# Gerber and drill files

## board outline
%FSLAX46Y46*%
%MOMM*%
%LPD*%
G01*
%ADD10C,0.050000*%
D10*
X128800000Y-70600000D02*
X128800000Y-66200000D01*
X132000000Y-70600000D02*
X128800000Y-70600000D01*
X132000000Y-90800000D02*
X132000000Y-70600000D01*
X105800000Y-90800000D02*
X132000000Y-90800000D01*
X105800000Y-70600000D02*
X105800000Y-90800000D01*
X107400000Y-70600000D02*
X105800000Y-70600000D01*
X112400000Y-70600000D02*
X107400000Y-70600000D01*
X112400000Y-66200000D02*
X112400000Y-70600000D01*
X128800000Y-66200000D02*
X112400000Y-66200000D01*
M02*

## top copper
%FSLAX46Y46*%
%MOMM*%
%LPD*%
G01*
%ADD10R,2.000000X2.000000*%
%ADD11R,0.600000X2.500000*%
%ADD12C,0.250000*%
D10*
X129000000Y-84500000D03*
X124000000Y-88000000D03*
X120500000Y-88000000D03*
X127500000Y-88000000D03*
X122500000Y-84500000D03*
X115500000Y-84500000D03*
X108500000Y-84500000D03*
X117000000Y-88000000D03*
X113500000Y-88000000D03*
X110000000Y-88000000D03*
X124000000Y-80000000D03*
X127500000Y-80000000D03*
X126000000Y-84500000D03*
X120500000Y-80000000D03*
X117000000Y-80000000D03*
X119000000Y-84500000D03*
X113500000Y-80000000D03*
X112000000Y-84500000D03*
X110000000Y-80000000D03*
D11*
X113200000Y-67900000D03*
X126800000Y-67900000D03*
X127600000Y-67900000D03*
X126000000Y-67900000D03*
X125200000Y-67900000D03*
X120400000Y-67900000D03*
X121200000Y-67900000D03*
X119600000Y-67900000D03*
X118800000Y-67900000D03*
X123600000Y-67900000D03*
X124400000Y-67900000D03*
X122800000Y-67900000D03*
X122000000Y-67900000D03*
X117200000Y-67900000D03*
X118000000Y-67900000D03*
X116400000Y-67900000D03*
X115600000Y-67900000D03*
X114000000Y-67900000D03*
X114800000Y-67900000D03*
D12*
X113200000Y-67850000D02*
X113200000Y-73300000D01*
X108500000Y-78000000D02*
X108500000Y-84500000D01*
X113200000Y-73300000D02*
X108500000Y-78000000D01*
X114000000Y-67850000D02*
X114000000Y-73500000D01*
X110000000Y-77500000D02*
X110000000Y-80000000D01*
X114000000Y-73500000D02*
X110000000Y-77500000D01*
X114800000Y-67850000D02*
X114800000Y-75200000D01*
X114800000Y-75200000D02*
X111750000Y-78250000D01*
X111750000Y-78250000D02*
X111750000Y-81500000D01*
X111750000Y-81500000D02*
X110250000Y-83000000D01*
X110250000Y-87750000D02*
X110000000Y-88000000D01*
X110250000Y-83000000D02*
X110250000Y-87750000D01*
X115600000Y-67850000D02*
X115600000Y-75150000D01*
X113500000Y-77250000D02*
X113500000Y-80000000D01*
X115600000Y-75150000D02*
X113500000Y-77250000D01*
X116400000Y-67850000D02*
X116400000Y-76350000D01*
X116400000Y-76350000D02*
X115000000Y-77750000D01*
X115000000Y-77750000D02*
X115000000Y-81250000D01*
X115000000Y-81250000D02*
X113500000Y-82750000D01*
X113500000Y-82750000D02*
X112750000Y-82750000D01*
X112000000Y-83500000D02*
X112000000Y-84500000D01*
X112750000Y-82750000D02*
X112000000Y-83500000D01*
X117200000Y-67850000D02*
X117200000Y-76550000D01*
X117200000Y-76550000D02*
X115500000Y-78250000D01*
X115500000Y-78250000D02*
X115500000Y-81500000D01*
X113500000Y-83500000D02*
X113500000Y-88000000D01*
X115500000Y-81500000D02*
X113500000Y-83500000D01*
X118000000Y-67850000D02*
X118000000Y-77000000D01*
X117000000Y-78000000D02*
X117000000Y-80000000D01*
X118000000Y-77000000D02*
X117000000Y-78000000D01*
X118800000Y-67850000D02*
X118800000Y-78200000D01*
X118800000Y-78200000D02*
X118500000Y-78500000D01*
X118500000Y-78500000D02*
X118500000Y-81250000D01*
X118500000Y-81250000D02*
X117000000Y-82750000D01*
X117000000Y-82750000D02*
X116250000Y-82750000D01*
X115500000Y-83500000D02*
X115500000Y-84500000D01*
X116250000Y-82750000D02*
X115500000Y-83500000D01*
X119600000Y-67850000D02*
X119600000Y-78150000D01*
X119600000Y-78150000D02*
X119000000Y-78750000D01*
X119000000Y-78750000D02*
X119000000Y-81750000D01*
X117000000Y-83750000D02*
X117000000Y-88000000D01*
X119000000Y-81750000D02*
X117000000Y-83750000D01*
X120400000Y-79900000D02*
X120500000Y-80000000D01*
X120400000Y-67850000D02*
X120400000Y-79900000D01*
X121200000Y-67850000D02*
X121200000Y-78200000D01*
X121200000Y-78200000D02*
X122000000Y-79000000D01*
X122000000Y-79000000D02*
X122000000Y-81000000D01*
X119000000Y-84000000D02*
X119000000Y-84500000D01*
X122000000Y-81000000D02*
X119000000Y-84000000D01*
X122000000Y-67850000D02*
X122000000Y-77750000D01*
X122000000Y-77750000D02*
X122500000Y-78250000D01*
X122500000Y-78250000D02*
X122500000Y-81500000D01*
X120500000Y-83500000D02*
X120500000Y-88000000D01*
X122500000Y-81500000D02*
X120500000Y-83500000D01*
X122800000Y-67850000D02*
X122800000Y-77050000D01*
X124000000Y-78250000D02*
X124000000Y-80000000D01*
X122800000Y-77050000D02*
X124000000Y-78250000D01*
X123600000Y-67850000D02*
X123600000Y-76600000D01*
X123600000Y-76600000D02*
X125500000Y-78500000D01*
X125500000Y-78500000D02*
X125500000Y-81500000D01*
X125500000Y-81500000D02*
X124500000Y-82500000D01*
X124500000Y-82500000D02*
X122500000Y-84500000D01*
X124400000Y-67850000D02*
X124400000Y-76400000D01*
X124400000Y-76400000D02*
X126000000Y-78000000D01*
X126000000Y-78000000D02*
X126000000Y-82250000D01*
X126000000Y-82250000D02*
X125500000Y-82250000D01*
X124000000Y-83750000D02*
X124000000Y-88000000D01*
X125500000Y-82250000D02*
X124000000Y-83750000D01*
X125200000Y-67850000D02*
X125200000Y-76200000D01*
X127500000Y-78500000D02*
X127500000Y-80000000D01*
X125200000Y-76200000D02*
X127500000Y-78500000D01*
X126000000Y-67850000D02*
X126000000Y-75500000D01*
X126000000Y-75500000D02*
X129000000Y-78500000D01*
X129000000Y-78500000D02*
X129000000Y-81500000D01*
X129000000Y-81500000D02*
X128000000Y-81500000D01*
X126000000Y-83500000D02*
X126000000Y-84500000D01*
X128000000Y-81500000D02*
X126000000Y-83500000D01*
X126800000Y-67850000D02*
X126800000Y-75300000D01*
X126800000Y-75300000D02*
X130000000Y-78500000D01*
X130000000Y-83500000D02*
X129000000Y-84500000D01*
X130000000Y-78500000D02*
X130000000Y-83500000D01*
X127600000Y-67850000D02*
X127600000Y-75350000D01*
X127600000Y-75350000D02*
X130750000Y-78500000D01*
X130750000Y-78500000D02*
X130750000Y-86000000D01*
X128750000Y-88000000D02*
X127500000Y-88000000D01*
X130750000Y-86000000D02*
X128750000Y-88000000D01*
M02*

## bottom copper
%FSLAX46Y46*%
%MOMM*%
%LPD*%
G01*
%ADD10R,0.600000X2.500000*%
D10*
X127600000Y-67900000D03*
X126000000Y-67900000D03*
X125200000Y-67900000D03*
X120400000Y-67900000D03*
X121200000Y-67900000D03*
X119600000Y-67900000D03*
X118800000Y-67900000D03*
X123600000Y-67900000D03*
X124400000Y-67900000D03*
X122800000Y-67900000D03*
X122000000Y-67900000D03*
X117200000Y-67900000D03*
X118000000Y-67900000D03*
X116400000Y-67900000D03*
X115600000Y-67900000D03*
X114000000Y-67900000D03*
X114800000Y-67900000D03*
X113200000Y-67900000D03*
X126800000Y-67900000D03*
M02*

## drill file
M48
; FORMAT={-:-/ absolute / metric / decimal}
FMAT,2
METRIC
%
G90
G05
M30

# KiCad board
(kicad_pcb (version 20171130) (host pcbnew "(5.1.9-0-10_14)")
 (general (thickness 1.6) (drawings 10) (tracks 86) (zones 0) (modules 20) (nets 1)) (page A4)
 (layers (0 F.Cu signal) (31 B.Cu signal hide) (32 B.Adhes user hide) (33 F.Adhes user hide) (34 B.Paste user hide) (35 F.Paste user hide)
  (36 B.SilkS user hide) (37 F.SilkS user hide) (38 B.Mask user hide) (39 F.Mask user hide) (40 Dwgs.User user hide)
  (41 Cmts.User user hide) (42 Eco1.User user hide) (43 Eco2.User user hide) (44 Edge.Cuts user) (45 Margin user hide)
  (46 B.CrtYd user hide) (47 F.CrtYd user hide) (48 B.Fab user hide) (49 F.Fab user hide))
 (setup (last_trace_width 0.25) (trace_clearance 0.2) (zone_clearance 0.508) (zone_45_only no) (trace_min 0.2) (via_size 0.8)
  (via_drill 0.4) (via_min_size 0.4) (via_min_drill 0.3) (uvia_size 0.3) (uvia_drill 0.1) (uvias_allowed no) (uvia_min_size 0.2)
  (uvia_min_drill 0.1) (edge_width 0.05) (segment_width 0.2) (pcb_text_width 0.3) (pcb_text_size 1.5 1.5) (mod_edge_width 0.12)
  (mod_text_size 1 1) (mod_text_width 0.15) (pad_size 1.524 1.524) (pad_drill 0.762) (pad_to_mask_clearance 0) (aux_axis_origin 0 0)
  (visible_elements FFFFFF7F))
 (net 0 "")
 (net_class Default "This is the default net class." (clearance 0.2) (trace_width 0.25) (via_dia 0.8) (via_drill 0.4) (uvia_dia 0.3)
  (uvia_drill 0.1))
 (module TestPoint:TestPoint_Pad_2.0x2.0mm (layer F.Cu) (at 129 84.5)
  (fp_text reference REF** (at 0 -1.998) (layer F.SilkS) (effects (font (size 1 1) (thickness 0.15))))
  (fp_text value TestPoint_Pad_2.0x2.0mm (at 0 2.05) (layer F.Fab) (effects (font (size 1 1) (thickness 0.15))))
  (pad 1 smd rect (at 0 0) (size 2 2) (layers F.Cu F.Mask)))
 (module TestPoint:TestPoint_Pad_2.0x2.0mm (layer F.Cu) (at 124 88)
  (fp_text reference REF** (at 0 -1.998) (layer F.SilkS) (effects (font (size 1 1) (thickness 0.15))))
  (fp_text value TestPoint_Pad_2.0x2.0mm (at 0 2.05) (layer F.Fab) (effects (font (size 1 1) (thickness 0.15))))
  (pad 1 smd rect (at 0 0) (size 2 2) (layers F.Cu F.Mask)))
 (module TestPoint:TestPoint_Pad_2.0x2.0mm (layer F.Cu) (at 120.5 88)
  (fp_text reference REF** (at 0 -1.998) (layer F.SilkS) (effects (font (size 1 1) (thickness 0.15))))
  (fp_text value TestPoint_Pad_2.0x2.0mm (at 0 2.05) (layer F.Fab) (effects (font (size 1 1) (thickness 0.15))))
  (pad 1 smd rect (at 0 0) (size 2 2) (layers F.Cu F.Mask)))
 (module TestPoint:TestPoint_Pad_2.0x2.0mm (layer F.Cu) (at 127.5 88)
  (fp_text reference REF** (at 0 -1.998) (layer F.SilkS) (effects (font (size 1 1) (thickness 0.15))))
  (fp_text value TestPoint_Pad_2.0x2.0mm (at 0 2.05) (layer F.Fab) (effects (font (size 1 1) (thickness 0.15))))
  (pad 1 smd rect (at 0 0) (size 2 2) (layers F.Cu F.Mask)))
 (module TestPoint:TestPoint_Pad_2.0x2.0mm (layer F.Cu) (at 122.5 84.5)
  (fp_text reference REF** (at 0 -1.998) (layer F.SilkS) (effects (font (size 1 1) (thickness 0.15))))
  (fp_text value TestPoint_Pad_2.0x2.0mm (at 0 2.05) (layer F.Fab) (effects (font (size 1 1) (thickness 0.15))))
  (pad 1 smd rect (at 0 0) (size 2 2) (layers F.Cu F.Mask)))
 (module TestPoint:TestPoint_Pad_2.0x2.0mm (layer F.Cu) (at 115.5 84.5)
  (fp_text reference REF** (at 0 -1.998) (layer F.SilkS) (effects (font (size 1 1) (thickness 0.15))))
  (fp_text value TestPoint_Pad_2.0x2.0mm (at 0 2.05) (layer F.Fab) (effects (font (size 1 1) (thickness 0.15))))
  (pad 1 smd rect (at 0 0) (size 2 2) (layers F.Cu F.Mask)))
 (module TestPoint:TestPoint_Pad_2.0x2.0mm (layer F.Cu) (at 108.5 84.5)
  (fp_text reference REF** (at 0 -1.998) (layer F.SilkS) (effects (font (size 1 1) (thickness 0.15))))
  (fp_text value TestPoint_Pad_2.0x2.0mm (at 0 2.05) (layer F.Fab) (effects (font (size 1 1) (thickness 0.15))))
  (pad 1 smd rect (at 0 0) (size 2 2) (layers F.Cu F.Mask)))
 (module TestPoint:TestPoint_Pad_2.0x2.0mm (layer F.Cu) (at 117 88)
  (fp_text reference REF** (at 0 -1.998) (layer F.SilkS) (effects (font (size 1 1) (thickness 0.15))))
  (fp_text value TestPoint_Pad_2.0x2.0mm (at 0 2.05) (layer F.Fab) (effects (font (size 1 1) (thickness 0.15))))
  (pad 1 smd rect (at 0 0) (size 2 2) (layers F.Cu F.Mask)))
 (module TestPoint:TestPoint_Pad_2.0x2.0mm (layer F.Cu) (at 113.5 88)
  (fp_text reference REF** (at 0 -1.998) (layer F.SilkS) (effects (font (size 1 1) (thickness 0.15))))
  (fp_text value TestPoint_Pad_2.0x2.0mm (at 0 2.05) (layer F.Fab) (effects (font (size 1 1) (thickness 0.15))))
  (pad 1 smd rect (at 0 0) (size 2 2) (layers F.Cu F.Mask)))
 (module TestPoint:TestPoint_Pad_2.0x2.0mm (layer F.Cu) (at 110 88)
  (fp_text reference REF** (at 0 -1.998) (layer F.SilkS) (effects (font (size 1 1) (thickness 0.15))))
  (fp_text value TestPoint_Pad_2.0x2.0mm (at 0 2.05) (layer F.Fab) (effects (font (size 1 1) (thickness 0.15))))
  (pad 1 smd rect (at 0 0) (size 2 2) (layers F.Cu F.Mask)))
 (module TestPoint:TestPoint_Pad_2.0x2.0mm (layer F.Cu) (at 124 80)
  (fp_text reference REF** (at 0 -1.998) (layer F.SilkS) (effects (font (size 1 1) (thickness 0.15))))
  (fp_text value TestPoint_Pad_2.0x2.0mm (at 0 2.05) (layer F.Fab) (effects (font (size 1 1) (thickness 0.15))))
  (pad 1 smd rect (at 0 0) (size 2 2) (layers F.Cu F.Mask)))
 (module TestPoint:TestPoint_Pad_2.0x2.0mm (layer F.Cu) (at 127.5 80)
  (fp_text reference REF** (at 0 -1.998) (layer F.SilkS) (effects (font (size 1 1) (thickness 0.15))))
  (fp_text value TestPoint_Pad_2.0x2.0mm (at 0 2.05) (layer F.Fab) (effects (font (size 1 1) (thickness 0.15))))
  (pad 1 smd rect (at 0 0) (size 2 2) (layers F.Cu F.Mask)))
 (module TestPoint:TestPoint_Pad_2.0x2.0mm (layer F.Cu) (at 126 84.5)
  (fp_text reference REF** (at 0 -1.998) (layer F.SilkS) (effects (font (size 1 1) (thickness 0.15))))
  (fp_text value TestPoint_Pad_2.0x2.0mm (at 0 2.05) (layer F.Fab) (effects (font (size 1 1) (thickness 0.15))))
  (pad 1 smd rect (at 0 0) (size 2 2) (layers F.Cu F.Mask)))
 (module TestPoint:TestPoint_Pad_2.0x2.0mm (layer F.Cu) (at 120.5 80)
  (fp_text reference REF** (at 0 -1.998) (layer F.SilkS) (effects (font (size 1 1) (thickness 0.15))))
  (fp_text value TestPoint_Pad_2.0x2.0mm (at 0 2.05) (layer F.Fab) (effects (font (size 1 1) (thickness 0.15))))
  (pad 1 smd rect (at 0 0) (size 2 2) (layers F.Cu F.Mask)))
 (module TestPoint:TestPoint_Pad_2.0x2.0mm (layer F.Cu) (at 117 80)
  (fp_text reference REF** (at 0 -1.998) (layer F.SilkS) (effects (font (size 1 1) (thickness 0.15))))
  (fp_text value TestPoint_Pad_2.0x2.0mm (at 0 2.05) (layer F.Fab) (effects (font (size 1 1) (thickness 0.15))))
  (pad 1 smd rect (at 0 0) (size 2 2) (layers F.Cu F.Mask)))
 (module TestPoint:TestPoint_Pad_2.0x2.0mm (layer F.Cu) (at 119 84.5)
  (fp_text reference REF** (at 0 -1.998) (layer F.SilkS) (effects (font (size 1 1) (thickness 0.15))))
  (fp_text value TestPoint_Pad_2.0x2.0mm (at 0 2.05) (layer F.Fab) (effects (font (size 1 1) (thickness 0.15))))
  (pad 1 smd rect (at 0 0) (size 2 2) (layers F.Cu F.Mask)))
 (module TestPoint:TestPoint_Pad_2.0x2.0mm (layer F.Cu) (at 113.5 80)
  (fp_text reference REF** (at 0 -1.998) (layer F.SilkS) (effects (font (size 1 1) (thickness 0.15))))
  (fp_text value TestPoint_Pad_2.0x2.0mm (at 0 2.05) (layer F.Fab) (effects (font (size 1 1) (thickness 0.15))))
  (pad 1 smd rect (at 0 0) (size 2 2) (layers F.Cu F.Mask)))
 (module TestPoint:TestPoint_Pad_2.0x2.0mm (layer F.Cu) (at 112 84.5)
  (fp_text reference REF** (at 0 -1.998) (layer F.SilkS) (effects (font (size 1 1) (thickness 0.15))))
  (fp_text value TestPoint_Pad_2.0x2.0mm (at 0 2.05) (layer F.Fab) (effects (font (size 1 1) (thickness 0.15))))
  (pad 1 smd rect (at 0 0) (size 2 2) (layers F.Cu F.Mask)))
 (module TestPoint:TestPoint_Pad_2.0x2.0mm (layer F.Cu) (at 110 80)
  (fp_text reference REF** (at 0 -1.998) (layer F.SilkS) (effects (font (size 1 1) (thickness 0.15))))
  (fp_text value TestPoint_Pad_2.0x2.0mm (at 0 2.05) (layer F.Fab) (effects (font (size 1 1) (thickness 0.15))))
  (pad 1 smd rect (at 0 0) (size 2 2) (layers F.Cu F.Mask)))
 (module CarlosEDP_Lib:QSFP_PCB (layer F.Cu) (at 112.8 69.45)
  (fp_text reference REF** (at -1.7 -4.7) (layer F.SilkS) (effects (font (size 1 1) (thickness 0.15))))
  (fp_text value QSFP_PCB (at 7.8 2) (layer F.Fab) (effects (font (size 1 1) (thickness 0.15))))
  (pad 1 smd rect (at 14.8 -1.5) (size 0.6 2.5) (drill (offset 0 -0.05)) (layers B.Cu B.Paste B.Mask))
  (pad 3 smd rect (at 13.2 -1.5) (size 0.6 2.5) (drill (offset 0 -0.05)) (layers B.Cu B.Paste B.Mask))
  (pad 4 smd rect (at 12.4 -1.5) (size 0.6 2.5) (drill (offset 0 -0.05)) (layers B.Cu B.Paste B.Mask))
  (pad 10 smd rect (at 7.6 -1.5) (size 0.6 2.5) (drill (offset 0 -0.05)) (layers B.Cu B.Paste B.Mask))
  (pad 9 smd rect (at 8.4 -1.5) (size 0.6 2.5) (drill (offset 0 -0.05)) (layers B.Cu B.Paste B.Mask))
  (pad 11 smd rect (at 6.8 -1.5) (size 0.6 2.5) (drill (offset 0 -0.05)) (layers B.Cu B.Paste B.Mask))
  (pad 12 smd rect (at 6 -1.5) (size 0.6 2.5) (drill (offset 0 -0.05)) (layers B.Cu B.Paste B.Mask))
  (pad 6 smd rect (at 10.8 -1.5) (size 0.6 2.5) (drill (offset 0 -0.05)) (layers B.Cu B.Paste B.Mask))
  (pad 5 smd rect (at 11.6 -1.5) (size 0.6 2.5) (drill (offset 0 -0.05)) (layers B.Cu B.Paste B.Mask))
  (pad 7 smd rect (at 10 -1.5) (size 0.6 2.5) (drill (offset 0 -0.05)) (layers B.Cu B.Paste B.Mask))
  (pad 8 smd rect (at 9.2 -1.5) (size 0.6 2.5) (drill (offset 0 -0.05)) (layers B.Cu B.Paste B.Mask))
  (pad 14 smd rect (at 4.4 -1.5) (size 0.6 2.5) (drill (offset 0 -0.05)) (layers B.Cu B.Paste B.Mask))
  (pad 13 smd rect (at 5.2 -1.5) (size 0.6 2.5) (drill (offset 0 -0.05)) (layers B.Cu B.Paste B.Mask))
  (pad 15 smd rect (at 3.6 -1.5) (size 0.6 2.5) (drill (offset 0 -0.05)) (layers B.Cu B.Paste B.Mask))
  (pad 16 smd rect (at 2.8 -1.5) (size 0.6 2.5) (drill (offset 0 -0.05)) (layers B.Cu B.Paste B.Mask))
  (pad 18 smd rect (at 1.2 -1.5) (size 0.6 2.5) (drill (offset 0 -0.05)) (layers B.Cu B.Paste B.Mask))
  (pad 17 smd rect (at 2 -1.5) (size 0.6 2.5) (drill (offset 0 -0.05)) (layers B.Cu B.Paste B.Mask))
  (pad 19 smd rect (at 0.4 -1.5) (size 0.6 2.5) (drill (offset 0 -0.05)) (layers B.Cu B.Paste B.Mask))
  (pad 2 smd rect (at 14 -1.5) (size 0.6 2.5) (drill (offset 0 -0.05)) (layers B.Cu B.Paste B.Mask))
  (pad 38 smd rect (at 0.4 -1.6) (size 0.6 2.5) (drill (offset 0 0.05)) (layers F.Cu F.Paste F.Mask))
  (pad 21 smd rect (at 14 -1.6) (size 0.6 2.5) (drill (offset 0 0.05)) (layers F.Cu F.Paste F.Mask))
  (pad 20 smd rect (at 14.8 -1.6) (size 0.6 2.5) (drill (offset 0 0.05)) (layers F.Cu F.Paste F.Mask))
  (pad 22 smd rect (at 13.2 -1.6) (size 0.6 2.5) (drill (offset 0 0.05)) (layers F.Cu F.Paste F.Mask))
  (pad 23 smd rect (at 12.4 -1.6) (size 0.6 2.5) (drill (offset 0 0.05)) (layers F.Cu F.Paste F.Mask))
  (pad 29 smd rect (at 7.6 -1.6) (size 0.6 2.5) (drill (offset 0 0.05)) (layers F.Cu F.Paste F.Mask))
  (pad 28 smd rect (at 8.4 -1.6) (size 0.6 2.5) (drill (offset 0 0.05)) (layers F.Cu F.Paste F.Mask))
  (pad 30 smd rect (at 6.8 -1.6) (size 0.6 2.5) (drill (offset 0 0.05)) (layers F.Cu F.Paste F.Mask))
  (pad 31 smd rect (at 6 -1.6) (size 0.6 2.5) (drill (offset 0 0.05)) (layers F.Cu F.Paste F.Mask))
  (pad 25 smd rect (at 10.8 -1.6) (size 0.6 2.5) (drill (offset 0 0.05)) (layers F.Cu F.Paste F.Mask))
  (pad 24 smd rect (at 11.6 -1.6) (size 0.6 2.5) (drill (offset 0 0.05)) (layers F.Cu F.Paste F.Mask))
  (pad 26 smd rect (at 10 -1.6) (size 0.6 2.5) (drill (offset 0 0.05)) (layers F.Cu F.Paste F.Mask))
  (pad 27 smd rect (at 9.2 -1.6) (size 0.6 2.5) (drill (offset 0 0.05)) (layers F.Cu F.Paste F.Mask))
  (pad 33 smd rect (at 4.4 -1.6) (size 0.6 2.5) (drill (offset 0 0.05)) (layers F.Cu F.Paste F.Mask))
  (pad 32 smd rect (at 5.2 -1.6) (size 0.6 2.5) (drill (offset 0 0.05)) (layers F.Cu F.Paste F.Mask))
  (pad 34 smd rect (at 3.6 -1.6) (size 0.6 2.5) (drill (offset 0 0.05)) (layers F.Cu F.Paste F.Mask))
  (pad 35 smd rect (at 2.8 -1.6) (size 0.6 2.5) (drill (offset 0 0.05)) (layers F.Cu F.Paste F.Mask))
  (pad 37 smd rect (at 1.2 -1.6) (size 0.6 2.5) (drill (offset 0 0.05)) (layers F.Cu F.Paste F.Mask))
  (pad 36 smd rect (at 2 -1.6) (size 0.6 2.5) (drill (offset 0 0.05)) (layers F.Cu F.Paste F.Mask)))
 (gr_line (start 128.8 70.6) (end 128.8 66.2) (layer Edge.Cuts) (width 0.05))
 (gr_line (start 132 70.6) (end 128.8 70.6) (layer Edge.Cuts) (width 0.05))
 (gr_line (start 132 90.8) (end 132 70.6) (layer Edge.Cuts) (width 0.05))
 (gr_line (start 105.8 90.8) (end 132 90.8) (layer Edge.Cuts) (width 0.05))
 (gr_line (start 105.8 70.6) (end 105.8 90.8) (layer Edge.Cuts) (width 0.05))
 (gr_line (start 107.4 70.6) (end 105.8 70.6) (layer Edge.Cuts) (width 0.05))
 (gr_line (start 112.4 70.6) (end 107.4 70.6) (layer Edge.Cuts) (width 0.05))
 (gr_line (start 112.4 66.2) (end 112.4 70.6) (layer Edge.Cuts) (width 0.05))
 (gr_line (start 128.8 66.2) (end 112.4 66.2) (layer Edge.Cuts) (width 0.05))
 (segment (start 113.2 67.85) (end 113.2 73.3) (width 0.25) (layer F.Cu) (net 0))
 (segment (start 108.5 78) (end 108.5 84.5) (width 0.25) (layer F.Cu) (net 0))
 (segment (start 113.2 73.3) (end 108.5 78) (width 0.25) (layer F.Cu) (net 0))
 (segment (start 114 67.85) (end 114 73.5) (width 0.25) (layer F.Cu) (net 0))
 (segment (start 110 77.5) (end 110 80) (width 0.25) (layer F.Cu) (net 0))
 (segment (start 114 73.5) (end 110 77.5) (width 0.25) (layer F.Cu) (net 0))
 (segment (start 114.8 67.85) (end 114.8 75.2) (width 0.25) (layer F.Cu) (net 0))
 (segment (start 114.8 75.2) (end 111.75 78.25) (width 0.25) (layer F.Cu) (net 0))
 (segment (start 111.75 78.25) (end 111.75 81.5) (width 0.25) (layer F.Cu) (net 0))
 (segment (start 111.75 81.5) (end 110.25 83) (width 0.25) (layer F.Cu) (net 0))
 (segment (start 110.25 87.75) (end 110 88) (width 0.25) (layer F.Cu) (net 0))
 (segment (start 110.25 83) (end 110.25 87.75) (width 0.25) (layer F.Cu) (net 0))
 (segment (start 115.6 67.85) (end 115.6 75.15) (width 0.25) (layer F.Cu) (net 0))
 (segment (start 113.5 77.25) (end 113.5 80) (width 0.25) (layer F.Cu) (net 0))
 (segment (start 115.6 75.15) (end 113.5 77.25) (width 0.25) (layer F.Cu) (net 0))
 (segment (start 116.4 67.85) (end 116.4 76.35) (width 0.25) (layer F.Cu) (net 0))
 (segment (start 116.4 76.35) (end 115 77.75) (width 0.25) (layer F.Cu) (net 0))
 (segment (start 115 77.75) (end 115 81.25) (width 0.25) (layer F.Cu) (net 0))
 (segment (start 115 81.25) (end 113.5 82.75) (width 0.25) (layer F.Cu) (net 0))
 (segment (start 113.5 82.75) (end 112.75 82.75) (width 0.25) (layer F.Cu) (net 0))
 (segment (start 112 83.5) (end 112 84.5) (width 0.25) (layer F.Cu) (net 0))
 (segment (start 112.75 82.75) (end 112 83.5) (width 0.25) (layer F.Cu) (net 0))
 (segment (start 117.2 67.85) (end 117.2 76.55) (width 0.25) (layer F.Cu) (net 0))
 (segment (start 117.2 76.55) (end 115.5 78.25) (width 0.25) (layer F.Cu) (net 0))
 (segment (start 115.5 78.25) (end 115.5 81.5) (width 0.25) (layer F.Cu) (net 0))
 (segment (start 113.5 83.5) (end 113.5 88) (width 0.25) (layer F.Cu) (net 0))
 (segment (start 115.5 81.5) (end 113.5 83.5) (width 0.25) (layer F.Cu) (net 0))
 (segment (start 118 67.85) (end 118 77) (width 0.25) (layer F.Cu) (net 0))
 (segment (start 117 78) (end 117 80) (width 0.25) (layer F.Cu) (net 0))
 (segment (start 118 77) (end 117 78) (width 0.25) (layer F.Cu) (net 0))
 (segment (start 118.8 67.85) (end 118.8 78.2) (width 0.25) (layer F.Cu) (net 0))
 (segment (start 118.8 78.2) (end 118.5 78.5) (width 0.25) (layer F.Cu) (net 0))
 (segment (start 118.5 78.5) (end 118.5 81.25) (width 0.25) (layer F.Cu) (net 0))
 (segment (start 118.5 81.25) (end 117 82.75) (width 0.25) (layer F.Cu) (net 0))
 (segment (start 117 82.75) (end 116.25 82.75) (width 0.25) (layer F.Cu) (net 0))
 (segment (start 115.5 83.5) (end 115.5 84.5) (width 0.25) (layer F.Cu) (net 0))
 (segment (start 116.25 82.75) (end 115.5 83.5) (width 0.25) (layer F.Cu) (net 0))
 (segment (start 119.6 67.85) (end 119.6 78.15) (width 0.25) (layer F.Cu) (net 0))
 (segment (start 119.6 78.15) (end 119 78.75) (width 0.25) (layer F.Cu) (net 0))
 (segment (start 119 78.75) (end 119 81.75) (width 0.25) (layer F.Cu) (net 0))
 (segment (start 117 83.75) (end 117 88) (width 0.25) (layer F.Cu) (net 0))
 (segment (start 119 81.75) (end 117 83.75) (width 0.25) (layer F.Cu) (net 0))
 (segment (start 120.4 79.9) (end 120.5 80) (width 0.25) (layer F.Cu) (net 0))
 (segment (start 120.4 67.85) (end 120.4 79.9) (width 0.25) (layer F.Cu) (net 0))
 (segment (start 121.2 67.85) (end 121.2 78.2) (width 0.25) (layer F.Cu) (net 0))
 (segment (start 121.2 78.2) (end 122 79) (width 0.25) (layer F.Cu) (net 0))
 (segment (start 122 79) (end 122 81) (width 0.25) (layer F.Cu) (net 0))
 (segment (start 119 84) (end 119 84.5) (width 0.25) (layer F.Cu) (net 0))
 (segment (start 122 81) (end 119 84) (width 0.25) (layer F.Cu) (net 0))
 (segment (start 122 67.85) (end 122 77.75) (width 0.25) (layer F.Cu) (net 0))
 (segment (start 122 77.75) (end 122.5 78.25) (width 0.25) (layer F.Cu) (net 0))
 (segment (start 122.5 78.25) (end 122.5 81.5) (width 0.25) (layer F.Cu) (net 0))
 (segment (start 120.5 83.5) (end 120.5 88) (width 0.25) (layer F.Cu) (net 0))
 (segment (start 122.5 81.5) (end 120.5 83.5) (width 0.25) (layer F.Cu) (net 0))
 (segment (start 122.8 67.85) (end 122.8 77.05) (width 0.25) (layer F.Cu) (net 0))
 (segment (start 124 78.25) (end 124 80) (width 0.25) (layer F.Cu) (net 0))
 (segment (start 122.8 77.05) (end 124 78.25) (width 0.25) (layer F.Cu) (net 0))
 (segment (start 123.6 67.85) (end 123.6 76.6) (width 0.25) (layer F.Cu) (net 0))
 (segment (start 123.6 76.6) (end 125.5 78.5) (width 0.25) (layer F.Cu) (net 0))
 (segment (start 125.5 78.5) (end 125.5 81.5) (width 0.25) (layer F.Cu) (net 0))
 (segment (start 125.5 81.5) (end 124.5 82.5) (width 0.25) (layer F.Cu) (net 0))
 (segment (start 124.5 82.5) (end 122.5 84.5) (width 0.25) (layer F.Cu) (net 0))
 (segment (start 124.4 67.85) (end 124.4 76.4) (width 0.25) (layer F.Cu) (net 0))
 (segment (start 124.4 76.4) (end 126 78) (width 0.25) (layer F.Cu) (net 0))
 (segment (start 126 78) (end 126 82.25) (width 0.25) (layer F.Cu) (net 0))
 (segment (start 126 82.25) (end 125.5 82.25) (width 0.25) (layer F.Cu) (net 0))
 (segment (start 124 83.75) (end 124 88) (width 0.25) (layer F.Cu) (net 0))
 (segment (start 125.5 82.25) (end 124 83.75) (width 0.25) (layer F.Cu) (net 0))
 (segment (start 125.2 67.85) (end 125.2 76.2) (width 0.25) (layer F.Cu) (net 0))
 (segment (start 127.5 78.5) (end 127.5 80) (width 0.25) (layer F.Cu) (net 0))
 (segment (start 125.2 76.2) (end 127.5 78.5) (width 0.25) (layer F.Cu) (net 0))
 (segment (start 126 67.85) (end 126 75.5) (width 0.25) (layer F.Cu) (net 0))
 (segment (start 126 75.5) (end 129 78.5) (width 0.25) (layer F.Cu) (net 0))
 (segment (start 129 78.5) (end 129 81.5) (width 0.25) (layer F.Cu) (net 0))
 (segment (start 129 81.5) (end 128 81.5) (width 0.25) (layer F.Cu) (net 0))
 (segment (start 126 83.5) (end 126 84.5) (width 0.25) (layer F.Cu) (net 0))
 (segment (start 128 81.5) (end 126 83.5) (width 0.25) (layer F.Cu) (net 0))
 (segment (start 126.8 67.85) (end 126.8 75.3) (width 0.25) (layer F.Cu) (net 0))
 (segment (start 126.8 75.3) (end 130 78.5) (width 0.25) (layer F.Cu) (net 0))
 (segment (start 130 83.5) (end 129 84.5) (width 0.25) (layer F.Cu) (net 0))
 (segment (start 130 78.5) (end 130 83.5) (width 0.25) (layer F.Cu) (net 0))
 (segment (start 127.6 67.85) (end 127.6 75.35) (width 0.25) (layer F.Cu) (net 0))
 (segment (start 127.6 75.35) (end 130.75 78.5) (width 0.25) (layer F.Cu) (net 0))
 (segment (start 130.75 78.5) (end 130.75 86) (width 0.25) (layer F.Cu) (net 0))
 (segment (start 128.75 88) (end 127.5 88) (width 0.25) (layer F.Cu) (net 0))
 (segment (start 130.75 86) (end 128.75 88) (width 0.25) (layer F.Cu) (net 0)))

